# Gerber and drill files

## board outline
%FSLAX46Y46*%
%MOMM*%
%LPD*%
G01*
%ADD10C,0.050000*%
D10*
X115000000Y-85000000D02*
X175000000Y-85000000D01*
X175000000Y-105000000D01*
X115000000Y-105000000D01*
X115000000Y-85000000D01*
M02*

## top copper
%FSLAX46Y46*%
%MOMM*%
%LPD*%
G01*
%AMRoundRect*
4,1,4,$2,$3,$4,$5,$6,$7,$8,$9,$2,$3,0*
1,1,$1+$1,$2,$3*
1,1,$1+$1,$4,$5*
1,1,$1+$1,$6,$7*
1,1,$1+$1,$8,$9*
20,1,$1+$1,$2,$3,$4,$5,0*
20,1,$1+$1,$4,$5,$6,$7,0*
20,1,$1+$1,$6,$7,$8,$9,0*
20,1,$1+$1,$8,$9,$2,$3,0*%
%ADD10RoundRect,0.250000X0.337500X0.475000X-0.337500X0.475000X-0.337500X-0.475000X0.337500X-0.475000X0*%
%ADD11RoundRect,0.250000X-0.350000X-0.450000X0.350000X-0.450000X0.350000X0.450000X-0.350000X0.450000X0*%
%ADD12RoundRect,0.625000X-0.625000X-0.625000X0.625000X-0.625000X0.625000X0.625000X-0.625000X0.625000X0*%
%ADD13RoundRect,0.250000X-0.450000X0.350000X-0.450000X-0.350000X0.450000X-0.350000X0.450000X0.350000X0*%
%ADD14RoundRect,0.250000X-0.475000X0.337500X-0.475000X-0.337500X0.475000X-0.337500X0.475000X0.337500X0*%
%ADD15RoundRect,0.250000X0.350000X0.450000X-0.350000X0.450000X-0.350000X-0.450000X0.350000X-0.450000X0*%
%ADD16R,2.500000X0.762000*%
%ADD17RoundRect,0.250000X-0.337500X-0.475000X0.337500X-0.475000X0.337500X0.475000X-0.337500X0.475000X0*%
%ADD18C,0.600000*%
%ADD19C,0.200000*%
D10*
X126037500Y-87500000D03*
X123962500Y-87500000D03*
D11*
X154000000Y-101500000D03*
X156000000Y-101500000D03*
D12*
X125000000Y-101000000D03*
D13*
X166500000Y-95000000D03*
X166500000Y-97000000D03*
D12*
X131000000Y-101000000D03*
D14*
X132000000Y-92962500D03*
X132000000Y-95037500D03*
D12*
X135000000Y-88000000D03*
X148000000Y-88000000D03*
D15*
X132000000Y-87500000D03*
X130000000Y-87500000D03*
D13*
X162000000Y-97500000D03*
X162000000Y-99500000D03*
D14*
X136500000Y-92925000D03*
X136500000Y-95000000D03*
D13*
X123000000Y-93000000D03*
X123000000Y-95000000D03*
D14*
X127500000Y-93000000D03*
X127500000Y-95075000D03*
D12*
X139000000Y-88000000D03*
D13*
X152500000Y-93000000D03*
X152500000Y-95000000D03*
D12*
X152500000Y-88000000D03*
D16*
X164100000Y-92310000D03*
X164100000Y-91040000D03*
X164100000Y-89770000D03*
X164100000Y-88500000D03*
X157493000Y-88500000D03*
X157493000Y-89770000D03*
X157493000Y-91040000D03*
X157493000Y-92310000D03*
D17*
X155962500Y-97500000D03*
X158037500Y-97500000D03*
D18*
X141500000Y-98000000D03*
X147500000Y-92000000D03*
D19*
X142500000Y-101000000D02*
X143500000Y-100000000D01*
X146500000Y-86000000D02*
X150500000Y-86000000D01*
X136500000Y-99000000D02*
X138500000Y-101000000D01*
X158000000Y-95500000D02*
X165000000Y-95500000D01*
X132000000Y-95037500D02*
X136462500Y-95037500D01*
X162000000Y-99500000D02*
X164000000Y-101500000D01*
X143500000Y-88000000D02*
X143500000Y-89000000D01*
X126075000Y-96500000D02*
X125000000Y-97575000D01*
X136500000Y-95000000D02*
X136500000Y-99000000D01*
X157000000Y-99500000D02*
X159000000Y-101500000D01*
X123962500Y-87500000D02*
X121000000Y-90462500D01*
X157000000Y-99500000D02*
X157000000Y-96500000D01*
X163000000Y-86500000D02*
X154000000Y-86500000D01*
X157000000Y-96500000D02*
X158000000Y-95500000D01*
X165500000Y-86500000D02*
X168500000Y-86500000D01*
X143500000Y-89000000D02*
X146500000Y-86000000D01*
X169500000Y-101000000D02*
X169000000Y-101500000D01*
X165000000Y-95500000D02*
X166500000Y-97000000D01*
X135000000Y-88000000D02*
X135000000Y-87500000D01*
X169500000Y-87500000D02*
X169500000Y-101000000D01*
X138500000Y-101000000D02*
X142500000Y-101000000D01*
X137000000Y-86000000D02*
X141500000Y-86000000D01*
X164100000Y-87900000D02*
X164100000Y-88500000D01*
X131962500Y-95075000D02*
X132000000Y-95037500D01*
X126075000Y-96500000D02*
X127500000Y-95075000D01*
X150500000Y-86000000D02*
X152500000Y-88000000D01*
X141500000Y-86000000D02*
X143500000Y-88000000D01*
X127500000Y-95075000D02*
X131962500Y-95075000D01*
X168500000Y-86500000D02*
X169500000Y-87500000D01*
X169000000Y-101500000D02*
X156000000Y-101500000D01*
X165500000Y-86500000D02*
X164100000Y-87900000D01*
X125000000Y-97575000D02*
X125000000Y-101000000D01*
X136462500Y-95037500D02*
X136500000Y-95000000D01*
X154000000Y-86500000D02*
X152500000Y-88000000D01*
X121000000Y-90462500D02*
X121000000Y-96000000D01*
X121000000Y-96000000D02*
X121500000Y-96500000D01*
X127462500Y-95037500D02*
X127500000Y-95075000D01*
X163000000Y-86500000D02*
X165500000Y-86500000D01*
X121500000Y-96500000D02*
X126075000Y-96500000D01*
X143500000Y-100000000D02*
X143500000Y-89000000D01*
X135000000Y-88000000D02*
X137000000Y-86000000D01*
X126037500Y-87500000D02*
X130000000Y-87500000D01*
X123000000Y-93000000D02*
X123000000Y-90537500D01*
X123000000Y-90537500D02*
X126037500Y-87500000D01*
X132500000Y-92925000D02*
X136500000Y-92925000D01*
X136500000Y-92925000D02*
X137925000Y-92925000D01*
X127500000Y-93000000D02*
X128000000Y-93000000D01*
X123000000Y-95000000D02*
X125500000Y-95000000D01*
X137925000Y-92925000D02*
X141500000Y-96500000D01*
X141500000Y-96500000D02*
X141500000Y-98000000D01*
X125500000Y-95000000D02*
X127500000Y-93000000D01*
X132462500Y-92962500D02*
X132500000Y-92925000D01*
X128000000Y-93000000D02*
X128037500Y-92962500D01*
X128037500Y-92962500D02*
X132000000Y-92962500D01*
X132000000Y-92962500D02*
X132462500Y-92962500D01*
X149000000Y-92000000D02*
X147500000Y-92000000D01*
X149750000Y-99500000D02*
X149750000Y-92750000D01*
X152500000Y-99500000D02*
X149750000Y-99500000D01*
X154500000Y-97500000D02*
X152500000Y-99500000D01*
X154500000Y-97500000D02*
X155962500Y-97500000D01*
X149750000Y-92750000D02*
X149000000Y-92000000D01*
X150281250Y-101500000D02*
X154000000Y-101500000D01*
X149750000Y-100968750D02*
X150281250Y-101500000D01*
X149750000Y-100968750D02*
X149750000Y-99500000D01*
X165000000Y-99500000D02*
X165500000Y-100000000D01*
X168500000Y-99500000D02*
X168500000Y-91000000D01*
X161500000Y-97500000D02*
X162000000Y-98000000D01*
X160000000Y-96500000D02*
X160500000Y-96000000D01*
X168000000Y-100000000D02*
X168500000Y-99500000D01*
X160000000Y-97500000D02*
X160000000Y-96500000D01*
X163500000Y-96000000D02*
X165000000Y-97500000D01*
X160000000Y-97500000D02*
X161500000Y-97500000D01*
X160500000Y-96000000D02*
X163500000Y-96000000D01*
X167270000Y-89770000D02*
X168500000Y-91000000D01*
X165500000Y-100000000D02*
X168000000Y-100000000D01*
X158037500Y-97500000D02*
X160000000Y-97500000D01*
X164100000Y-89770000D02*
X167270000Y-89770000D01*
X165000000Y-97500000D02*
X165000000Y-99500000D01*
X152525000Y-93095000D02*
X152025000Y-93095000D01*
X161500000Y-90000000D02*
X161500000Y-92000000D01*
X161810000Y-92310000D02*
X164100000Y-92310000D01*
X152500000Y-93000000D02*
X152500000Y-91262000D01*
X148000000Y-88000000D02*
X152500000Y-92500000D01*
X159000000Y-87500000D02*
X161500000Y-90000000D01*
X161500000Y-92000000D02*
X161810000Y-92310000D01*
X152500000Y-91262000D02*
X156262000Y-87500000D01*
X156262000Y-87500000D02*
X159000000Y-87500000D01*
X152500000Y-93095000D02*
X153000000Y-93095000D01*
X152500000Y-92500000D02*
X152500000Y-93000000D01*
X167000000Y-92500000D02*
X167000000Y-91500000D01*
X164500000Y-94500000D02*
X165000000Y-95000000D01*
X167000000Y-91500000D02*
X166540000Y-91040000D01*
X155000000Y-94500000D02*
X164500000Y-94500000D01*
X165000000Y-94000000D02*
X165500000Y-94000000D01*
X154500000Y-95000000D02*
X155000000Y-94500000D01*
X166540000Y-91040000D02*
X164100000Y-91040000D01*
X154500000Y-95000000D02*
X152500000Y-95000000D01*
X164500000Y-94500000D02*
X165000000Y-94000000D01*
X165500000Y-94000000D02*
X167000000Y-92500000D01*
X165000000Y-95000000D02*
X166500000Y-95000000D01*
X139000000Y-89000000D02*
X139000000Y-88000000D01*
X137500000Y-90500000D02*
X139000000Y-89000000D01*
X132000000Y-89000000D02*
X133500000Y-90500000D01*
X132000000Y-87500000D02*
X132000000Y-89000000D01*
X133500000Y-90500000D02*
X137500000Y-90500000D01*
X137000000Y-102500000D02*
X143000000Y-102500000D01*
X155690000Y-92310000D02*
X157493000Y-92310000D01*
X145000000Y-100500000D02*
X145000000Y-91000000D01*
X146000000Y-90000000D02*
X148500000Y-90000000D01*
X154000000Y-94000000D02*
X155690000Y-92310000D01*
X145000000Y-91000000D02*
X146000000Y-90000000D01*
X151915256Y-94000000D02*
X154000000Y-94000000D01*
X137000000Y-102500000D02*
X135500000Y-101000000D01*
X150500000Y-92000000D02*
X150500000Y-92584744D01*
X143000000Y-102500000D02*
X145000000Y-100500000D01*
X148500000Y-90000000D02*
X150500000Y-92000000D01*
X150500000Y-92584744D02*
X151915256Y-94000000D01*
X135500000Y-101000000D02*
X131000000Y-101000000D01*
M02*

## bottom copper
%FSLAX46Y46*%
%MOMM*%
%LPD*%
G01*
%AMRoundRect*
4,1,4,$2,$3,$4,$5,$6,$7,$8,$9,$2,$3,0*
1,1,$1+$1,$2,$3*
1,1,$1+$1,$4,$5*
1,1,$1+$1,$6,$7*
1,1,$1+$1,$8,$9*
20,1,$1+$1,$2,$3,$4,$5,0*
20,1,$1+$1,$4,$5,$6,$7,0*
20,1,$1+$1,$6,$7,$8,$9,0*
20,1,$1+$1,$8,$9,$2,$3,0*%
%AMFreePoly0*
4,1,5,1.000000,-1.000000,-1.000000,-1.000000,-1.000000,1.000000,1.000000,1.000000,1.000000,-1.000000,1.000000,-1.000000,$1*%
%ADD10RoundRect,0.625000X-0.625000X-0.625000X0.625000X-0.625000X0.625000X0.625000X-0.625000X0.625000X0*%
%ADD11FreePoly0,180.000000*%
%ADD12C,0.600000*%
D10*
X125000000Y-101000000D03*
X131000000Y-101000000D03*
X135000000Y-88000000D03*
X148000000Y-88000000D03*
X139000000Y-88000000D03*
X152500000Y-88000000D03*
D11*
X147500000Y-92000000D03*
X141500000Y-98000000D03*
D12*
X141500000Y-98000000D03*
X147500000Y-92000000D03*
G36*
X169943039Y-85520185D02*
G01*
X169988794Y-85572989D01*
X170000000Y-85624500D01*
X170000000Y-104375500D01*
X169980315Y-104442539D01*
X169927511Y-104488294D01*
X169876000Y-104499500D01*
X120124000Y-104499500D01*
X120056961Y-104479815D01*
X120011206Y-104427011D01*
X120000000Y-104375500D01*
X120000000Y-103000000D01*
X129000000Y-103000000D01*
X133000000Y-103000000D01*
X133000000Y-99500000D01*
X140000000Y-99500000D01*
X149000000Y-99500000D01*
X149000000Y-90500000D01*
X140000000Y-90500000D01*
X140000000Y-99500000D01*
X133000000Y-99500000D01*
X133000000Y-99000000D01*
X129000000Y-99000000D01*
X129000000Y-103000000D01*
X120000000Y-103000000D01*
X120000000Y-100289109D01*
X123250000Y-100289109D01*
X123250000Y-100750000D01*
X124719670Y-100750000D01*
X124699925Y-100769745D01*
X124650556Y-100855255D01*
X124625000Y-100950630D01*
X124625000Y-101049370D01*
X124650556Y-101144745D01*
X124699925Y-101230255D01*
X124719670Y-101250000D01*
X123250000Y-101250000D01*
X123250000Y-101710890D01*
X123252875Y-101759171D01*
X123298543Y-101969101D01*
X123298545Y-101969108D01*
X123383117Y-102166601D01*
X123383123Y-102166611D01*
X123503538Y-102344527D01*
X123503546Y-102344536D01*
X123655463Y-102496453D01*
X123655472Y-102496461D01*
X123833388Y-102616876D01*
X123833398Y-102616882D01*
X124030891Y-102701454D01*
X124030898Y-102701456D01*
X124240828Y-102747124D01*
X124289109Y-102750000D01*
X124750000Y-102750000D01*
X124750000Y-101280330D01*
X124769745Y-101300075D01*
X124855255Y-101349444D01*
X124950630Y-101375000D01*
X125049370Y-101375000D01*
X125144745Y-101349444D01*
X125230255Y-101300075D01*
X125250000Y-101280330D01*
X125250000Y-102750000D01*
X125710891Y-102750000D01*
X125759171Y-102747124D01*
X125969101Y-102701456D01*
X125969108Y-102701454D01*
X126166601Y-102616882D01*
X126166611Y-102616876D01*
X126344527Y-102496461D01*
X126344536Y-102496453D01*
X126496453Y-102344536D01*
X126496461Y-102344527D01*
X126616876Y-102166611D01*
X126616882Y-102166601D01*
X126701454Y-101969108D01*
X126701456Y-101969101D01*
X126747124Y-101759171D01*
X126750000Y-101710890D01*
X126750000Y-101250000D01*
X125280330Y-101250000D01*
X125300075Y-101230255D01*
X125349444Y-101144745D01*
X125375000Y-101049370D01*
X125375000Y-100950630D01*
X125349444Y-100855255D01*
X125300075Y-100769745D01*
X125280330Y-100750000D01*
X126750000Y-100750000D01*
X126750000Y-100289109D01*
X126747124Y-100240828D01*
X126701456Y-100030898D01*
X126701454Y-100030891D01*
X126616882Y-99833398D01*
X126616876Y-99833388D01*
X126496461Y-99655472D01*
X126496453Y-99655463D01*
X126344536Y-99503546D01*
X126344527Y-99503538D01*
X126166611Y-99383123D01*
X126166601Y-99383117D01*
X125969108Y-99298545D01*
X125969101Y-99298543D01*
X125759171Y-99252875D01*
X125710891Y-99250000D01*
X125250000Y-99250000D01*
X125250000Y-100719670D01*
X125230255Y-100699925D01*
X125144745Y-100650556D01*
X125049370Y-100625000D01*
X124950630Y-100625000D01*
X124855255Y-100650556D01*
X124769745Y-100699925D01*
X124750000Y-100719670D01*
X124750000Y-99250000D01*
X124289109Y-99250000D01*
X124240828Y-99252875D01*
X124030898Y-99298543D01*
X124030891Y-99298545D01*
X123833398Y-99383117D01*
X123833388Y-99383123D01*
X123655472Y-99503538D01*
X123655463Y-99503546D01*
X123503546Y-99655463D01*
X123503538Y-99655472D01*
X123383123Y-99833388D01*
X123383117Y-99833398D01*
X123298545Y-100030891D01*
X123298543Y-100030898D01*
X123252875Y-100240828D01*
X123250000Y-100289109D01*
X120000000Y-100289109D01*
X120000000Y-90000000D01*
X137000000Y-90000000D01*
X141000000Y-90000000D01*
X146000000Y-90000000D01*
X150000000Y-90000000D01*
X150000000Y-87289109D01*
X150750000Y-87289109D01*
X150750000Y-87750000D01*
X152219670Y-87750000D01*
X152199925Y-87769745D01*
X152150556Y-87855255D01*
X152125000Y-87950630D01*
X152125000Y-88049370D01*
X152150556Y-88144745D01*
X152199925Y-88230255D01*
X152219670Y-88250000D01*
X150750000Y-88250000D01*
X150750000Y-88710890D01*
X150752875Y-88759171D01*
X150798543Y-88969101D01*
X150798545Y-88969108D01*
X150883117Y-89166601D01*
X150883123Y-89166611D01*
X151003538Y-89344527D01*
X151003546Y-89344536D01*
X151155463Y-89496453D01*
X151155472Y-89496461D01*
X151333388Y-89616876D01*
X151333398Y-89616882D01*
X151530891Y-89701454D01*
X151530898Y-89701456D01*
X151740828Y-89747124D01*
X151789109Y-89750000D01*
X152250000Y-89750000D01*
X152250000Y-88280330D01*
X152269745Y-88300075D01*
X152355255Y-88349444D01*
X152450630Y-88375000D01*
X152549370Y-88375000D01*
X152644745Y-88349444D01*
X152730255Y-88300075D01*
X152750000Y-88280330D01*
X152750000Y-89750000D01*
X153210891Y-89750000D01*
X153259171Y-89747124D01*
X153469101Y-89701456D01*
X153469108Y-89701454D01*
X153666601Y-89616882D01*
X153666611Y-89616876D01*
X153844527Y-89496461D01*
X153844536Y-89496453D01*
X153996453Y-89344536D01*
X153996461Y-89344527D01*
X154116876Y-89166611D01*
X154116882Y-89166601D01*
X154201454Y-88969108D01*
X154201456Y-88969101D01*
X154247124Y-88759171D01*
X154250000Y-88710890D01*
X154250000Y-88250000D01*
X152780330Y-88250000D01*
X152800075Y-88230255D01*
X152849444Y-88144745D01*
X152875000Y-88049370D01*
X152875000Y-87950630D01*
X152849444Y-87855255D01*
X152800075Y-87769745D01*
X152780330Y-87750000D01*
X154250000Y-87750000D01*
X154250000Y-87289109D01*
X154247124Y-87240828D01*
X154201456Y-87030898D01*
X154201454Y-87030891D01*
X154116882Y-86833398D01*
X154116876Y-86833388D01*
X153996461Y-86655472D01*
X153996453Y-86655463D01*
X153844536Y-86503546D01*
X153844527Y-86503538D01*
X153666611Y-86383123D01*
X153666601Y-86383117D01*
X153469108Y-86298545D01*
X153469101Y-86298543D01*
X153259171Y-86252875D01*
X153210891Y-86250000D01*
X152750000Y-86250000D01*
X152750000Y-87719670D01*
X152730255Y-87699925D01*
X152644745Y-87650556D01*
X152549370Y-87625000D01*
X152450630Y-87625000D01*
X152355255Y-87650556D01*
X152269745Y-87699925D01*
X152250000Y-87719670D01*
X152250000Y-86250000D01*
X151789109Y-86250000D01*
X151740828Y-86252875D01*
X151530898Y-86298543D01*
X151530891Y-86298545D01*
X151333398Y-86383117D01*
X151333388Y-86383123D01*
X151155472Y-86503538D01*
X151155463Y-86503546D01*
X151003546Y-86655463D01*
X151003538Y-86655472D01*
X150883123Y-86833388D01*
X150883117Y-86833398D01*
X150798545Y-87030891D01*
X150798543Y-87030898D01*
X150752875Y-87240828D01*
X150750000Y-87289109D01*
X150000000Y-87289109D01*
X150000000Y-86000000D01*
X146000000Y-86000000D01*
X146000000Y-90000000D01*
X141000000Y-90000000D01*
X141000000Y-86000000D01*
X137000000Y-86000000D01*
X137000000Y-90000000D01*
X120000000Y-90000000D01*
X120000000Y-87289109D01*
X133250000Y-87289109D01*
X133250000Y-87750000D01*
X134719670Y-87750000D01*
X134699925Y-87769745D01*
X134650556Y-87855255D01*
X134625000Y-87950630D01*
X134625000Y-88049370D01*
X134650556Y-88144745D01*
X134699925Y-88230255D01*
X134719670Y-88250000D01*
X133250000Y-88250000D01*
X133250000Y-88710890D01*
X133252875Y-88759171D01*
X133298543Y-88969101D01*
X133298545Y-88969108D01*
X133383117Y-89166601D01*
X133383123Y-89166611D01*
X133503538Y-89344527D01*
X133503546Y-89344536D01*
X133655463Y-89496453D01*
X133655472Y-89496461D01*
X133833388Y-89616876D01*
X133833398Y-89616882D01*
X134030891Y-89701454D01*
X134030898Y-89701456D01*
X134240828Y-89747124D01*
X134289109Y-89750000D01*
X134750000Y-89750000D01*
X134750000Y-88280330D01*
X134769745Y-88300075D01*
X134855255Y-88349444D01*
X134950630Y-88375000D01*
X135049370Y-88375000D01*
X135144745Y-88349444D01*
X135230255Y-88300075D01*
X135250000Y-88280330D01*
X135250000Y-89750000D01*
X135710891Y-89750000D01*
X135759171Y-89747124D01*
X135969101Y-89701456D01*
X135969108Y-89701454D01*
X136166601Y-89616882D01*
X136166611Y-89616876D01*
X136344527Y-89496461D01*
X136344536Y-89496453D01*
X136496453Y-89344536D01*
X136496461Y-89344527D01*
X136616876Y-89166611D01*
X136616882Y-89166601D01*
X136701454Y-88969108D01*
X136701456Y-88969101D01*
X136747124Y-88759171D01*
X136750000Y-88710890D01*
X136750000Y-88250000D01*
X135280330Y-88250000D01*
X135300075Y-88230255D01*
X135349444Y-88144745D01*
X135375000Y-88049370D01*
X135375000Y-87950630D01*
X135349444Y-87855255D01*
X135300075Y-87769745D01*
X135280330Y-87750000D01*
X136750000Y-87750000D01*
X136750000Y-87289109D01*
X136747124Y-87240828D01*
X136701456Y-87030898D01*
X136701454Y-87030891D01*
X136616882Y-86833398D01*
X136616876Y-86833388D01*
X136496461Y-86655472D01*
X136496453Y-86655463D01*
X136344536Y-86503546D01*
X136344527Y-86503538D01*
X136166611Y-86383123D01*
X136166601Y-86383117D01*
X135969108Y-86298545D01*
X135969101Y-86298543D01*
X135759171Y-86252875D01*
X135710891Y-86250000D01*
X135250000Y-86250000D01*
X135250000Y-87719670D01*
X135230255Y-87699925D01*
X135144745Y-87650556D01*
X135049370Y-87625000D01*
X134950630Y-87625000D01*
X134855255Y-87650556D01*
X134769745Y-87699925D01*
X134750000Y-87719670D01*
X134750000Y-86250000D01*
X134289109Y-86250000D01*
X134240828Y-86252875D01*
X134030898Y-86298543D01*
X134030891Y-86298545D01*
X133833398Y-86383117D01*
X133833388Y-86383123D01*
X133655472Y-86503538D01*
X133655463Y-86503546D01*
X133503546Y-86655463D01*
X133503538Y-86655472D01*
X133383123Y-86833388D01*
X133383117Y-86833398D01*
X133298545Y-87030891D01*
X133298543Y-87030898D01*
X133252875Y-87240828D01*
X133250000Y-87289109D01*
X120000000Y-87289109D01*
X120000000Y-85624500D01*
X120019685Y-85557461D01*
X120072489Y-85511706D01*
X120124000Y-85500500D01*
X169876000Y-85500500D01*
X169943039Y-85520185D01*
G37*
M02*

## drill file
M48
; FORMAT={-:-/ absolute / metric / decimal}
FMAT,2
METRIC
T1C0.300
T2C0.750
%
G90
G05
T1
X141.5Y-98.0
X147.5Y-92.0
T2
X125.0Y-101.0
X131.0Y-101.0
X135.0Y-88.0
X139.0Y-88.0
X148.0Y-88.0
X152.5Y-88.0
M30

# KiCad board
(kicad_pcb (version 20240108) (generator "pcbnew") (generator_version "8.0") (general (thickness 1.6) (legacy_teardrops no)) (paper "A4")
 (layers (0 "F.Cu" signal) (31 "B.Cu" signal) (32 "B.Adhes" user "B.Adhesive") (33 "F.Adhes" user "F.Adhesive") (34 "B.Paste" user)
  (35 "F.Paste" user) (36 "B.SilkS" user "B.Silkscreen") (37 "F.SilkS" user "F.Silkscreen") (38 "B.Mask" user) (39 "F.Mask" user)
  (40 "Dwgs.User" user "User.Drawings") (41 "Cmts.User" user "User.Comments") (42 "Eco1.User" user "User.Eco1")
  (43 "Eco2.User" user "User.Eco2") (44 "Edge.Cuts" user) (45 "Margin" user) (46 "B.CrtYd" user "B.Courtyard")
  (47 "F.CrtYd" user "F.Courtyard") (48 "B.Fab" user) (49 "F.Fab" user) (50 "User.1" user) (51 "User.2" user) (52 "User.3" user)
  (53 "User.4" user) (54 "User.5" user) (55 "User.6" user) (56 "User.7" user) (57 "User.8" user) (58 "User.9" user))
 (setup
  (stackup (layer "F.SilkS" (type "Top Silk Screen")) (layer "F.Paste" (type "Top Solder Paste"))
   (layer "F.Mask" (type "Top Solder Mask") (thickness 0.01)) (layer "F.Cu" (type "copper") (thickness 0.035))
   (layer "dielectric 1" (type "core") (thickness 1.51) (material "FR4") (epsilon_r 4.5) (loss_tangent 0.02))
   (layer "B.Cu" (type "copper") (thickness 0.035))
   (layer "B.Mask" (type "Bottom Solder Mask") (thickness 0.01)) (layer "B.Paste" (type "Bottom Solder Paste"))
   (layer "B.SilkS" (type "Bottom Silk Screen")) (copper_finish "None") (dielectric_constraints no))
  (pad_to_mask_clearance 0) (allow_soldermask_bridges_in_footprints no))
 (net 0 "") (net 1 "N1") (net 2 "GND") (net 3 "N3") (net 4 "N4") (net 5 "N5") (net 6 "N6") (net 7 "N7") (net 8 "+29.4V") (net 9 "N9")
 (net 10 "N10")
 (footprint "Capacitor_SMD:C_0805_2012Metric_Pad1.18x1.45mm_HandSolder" (layer "F.Cu") (at 125 87.5 180)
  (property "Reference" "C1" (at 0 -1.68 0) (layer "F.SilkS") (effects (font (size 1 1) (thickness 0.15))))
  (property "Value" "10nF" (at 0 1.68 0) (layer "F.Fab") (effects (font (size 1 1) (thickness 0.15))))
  (pad "1" smd roundrect (at -1.0375 0 180) (size 1.175 1.45) (layers "F.Cu" "F.Paste" "F.Mask") (roundrect_rratio 0.212766) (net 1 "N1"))
  (pad "2" smd roundrect (at 1.0375 0 180) (size 1.175 1.45) (layers "F.Cu" "F.Paste" "F.Mask") (roundrect_rratio 0.212766) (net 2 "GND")))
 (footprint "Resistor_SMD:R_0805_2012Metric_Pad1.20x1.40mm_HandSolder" (layer "F.Cu") (at 155 101.5)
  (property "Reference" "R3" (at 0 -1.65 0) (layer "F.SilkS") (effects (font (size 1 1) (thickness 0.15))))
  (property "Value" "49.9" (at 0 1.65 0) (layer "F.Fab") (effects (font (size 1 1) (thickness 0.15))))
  (pad "1" smd roundrect (at -1 0) (size 1.2 1.4) (layers "F.Cu" "F.Paste" "F.Mask") (roundrect_rratio 0.208333) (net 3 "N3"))
  (pad "2" smd roundrect (at 1 0) (size 1.2 1.4) (layers "F.Cu" "F.Paste" "F.Mask") (roundrect_rratio 0.208333) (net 2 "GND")))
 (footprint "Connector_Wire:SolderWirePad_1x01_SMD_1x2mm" (layer "F.Cu") (at 125 101)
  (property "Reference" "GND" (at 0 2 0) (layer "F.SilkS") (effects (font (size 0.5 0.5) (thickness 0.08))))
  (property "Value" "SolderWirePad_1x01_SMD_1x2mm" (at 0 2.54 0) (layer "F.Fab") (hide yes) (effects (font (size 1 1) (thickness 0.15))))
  (pad "1" thru_hole roundrect (at 0 0) (size 2.5 2.5) (drill 0.75) (layers "*.Cu" "*.Mask") (remove_unused_layers no)
   (roundrect_rratio 0.25) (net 2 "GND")))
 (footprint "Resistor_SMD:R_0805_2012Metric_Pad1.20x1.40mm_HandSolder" (layer "F.Cu") (at 166.5 96 -90)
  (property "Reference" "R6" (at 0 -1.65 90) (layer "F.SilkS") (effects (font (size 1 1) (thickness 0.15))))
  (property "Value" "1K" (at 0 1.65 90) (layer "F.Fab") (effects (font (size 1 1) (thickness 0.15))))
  (pad "1" smd roundrect (at -1 0 270) (size 1.2 1.4) (layers "F.Cu" "F.Paste" "F.Mask") (roundrect_rratio 0.208333) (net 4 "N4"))
  (pad "2" smd roundrect (at 1 0 270) (size 1.2 1.4) (layers "F.Cu" "F.Paste" "F.Mask") (roundrect_rratio 0.208333) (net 2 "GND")))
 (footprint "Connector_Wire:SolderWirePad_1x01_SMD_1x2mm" (layer "F.Cu") (at 131 101)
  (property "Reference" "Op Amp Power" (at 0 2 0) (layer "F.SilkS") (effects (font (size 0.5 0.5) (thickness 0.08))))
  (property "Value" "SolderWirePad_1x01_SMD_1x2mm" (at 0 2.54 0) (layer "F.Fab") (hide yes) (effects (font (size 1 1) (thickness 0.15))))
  (pad "1" thru_hole roundrect (at 0 0) (size 2.5 2.5) (drill 0.75) (layers "*.Cu" "*.Mask") (remove_unused_layers no)
   (roundrect_rratio 0.25) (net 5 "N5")))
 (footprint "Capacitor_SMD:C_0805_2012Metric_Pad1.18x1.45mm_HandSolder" (layer "F.Cu") (at 132 94 -90)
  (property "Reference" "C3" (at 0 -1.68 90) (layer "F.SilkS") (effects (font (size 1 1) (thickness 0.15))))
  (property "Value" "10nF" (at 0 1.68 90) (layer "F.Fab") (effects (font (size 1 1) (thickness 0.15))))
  (pad "1" smd roundrect (at -1.0375 0 270) (size 1.175 1.45) (layers "F.Cu" "F.Paste" "F.Mask") (roundrect_rratio 0.212766) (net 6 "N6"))
  (pad "2" smd roundrect (at 1.0375 0 270) (size 1.175 1.45) (layers "F.Cu" "F.Paste" "F.Mask") (roundrect_rratio 0.212766) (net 2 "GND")))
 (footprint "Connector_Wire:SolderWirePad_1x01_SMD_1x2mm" (layer "F.Cu") (at 135 88)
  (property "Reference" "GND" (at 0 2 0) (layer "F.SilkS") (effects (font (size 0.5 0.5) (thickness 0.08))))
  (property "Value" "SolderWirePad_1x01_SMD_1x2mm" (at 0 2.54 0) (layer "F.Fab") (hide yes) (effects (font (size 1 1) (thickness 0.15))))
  (pad "1" thru_hole roundrect (at 0 0) (size 2.5 2.5) (drill 0.75) (layers "*.Cu" "*.Mask") (remove_unused_layers no)
   (roundrect_rratio 0.25) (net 2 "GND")))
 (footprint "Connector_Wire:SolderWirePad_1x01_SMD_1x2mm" (layer "F.Cu") (at 148 88)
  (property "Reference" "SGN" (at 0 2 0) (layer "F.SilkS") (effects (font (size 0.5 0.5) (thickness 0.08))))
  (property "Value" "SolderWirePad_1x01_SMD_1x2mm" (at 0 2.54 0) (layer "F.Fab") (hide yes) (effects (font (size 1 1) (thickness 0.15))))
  (pad "1" thru_hole roundrect (at 0 0) (size 2.5 2.5) (drill 0.75) (layers "*.Cu" "*.Mask") (remove_unused_layers no)
   (roundrect_rratio 0.25) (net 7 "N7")))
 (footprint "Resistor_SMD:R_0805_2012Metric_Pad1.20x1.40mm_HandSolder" (layer "F.Cu") (at 131 87.5 180)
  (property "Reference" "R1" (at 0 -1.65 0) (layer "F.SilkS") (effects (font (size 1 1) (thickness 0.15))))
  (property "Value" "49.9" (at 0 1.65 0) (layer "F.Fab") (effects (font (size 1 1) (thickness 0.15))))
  (pad "1" smd roundrect (at -1 0 180) (size 1.2 1.4) (layers "F.Cu" "F.Paste" "F.Mask") (roundrect_rratio 0.208333) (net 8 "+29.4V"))
  (pad "2" smd roundrect (at 1 0 180) (size 1.2 1.4) (layers "F.Cu" "F.Paste" "F.Mask") (roundrect_rratio 0.208333) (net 1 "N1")))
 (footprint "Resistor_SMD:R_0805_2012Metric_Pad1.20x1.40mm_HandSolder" (layer "F.Cu") (at 162 98.5 -90)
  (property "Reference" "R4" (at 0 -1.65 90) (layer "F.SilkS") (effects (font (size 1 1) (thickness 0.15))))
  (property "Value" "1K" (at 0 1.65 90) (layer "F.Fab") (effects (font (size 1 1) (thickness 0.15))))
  (pad "1" smd roundrect (at -1 0 270) (size 1.2 1.4) (layers "F.Cu" "F.Paste" "F.Mask") (roundrect_rratio 0.208333) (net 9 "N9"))
  (pad "2" smd roundrect (at 1 0 270) (size 1.2 1.4) (layers "F.Cu" "F.Paste" "F.Mask") (roundrect_rratio 0.208333) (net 2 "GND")))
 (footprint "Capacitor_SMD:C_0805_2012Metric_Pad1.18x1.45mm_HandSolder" (layer "F.Cu") (at 136.5 93.9625 -90)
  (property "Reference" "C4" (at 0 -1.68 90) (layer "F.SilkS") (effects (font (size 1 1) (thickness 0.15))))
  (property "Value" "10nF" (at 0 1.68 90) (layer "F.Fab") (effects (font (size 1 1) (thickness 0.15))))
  (pad "1" smd roundrect (at -1.0375 0 270) (size 1.175 1.45) (layers "F.Cu" "F.Paste" "F.Mask") (roundrect_rratio 0.212766) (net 6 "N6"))
  (pad "2" smd roundrect (at 1.0375 0 270) (size 1.175 1.45) (layers "F.Cu" "F.Paste" "F.Mask") (roundrect_rratio 0.212766) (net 2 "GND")))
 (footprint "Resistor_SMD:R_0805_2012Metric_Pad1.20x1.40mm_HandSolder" (layer "F.Cu") (at 123 94 -90)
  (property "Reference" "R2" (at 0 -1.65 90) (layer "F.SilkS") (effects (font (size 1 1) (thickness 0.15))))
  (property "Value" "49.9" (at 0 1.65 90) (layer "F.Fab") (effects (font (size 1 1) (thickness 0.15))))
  (pad "1" smd roundrect (at -1 0 270) (size 1.2 1.4) (layers "F.Cu" "F.Paste" "F.Mask") (roundrect_rratio 0.208333) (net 1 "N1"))
  (pad "2" smd roundrect (at 1 0 270) (size 1.2 1.4) (layers "F.Cu" "F.Paste" "F.Mask") (roundrect_rratio 0.208333) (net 6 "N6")))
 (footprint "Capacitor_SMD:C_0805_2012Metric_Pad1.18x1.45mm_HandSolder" (layer "F.Cu") (at 127.5 94.0375 -90)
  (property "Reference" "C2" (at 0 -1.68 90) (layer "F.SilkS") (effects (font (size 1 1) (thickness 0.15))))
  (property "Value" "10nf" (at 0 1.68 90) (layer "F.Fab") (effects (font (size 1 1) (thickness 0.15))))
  (pad "1" smd roundrect (at -1.0375 0 270) (size 1.175 1.45) (layers "F.Cu" "F.Paste" "F.Mask") (roundrect_rratio 0.212766) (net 6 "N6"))
  (pad "2" smd roundrect (at 1.0375 0 270) (size 1.175 1.45) (layers "F.Cu" "F.Paste" "F.Mask") (roundrect_rratio 0.212766) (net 2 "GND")))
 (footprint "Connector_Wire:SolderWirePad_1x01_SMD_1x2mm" (layer "F.Cu") (at 139 88)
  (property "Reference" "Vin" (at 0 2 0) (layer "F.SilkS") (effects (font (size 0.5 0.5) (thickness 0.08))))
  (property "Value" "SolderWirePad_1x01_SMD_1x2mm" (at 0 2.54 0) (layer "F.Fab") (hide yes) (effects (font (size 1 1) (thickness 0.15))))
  (pad "1" thru_hole roundrect (at 0 0) (size 2.5 2.5) (drill 0.75) (layers "*.Cu" "*.Mask") (remove_unused_layers no)
   (roundrect_rratio 0.25) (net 8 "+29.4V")))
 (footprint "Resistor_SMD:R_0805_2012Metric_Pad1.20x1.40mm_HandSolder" (layer "F.Cu") (at 152.5 94 -90)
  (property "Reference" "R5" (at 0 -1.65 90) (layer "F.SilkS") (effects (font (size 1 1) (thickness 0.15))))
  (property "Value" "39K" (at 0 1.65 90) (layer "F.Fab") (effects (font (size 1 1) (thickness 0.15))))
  (pad "1" smd roundrect (at -1 0 270) (size 1.2 1.4) (layers "F.Cu" "F.Paste" "F.Mask") (roundrect_rratio 0.208333) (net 7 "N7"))
  (pad "2" smd roundrect (at 1 0 270) (size 1.2 1.4) (layers "F.Cu" "F.Paste" "F.Mask") (roundrect_rratio 0.208333) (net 4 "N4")))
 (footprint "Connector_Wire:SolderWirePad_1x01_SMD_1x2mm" (layer "F.Cu") (at 152.5 88)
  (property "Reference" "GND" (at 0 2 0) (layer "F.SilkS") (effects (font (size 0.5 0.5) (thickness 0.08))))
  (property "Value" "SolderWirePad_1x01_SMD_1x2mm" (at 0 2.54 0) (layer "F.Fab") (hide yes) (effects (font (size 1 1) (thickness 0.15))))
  (pad "1" thru_hole roundrect (at 0 0) (size 2.5 2.5) (drill 0.75) (layers "*.Cu" "*.Mask") (remove_unused_layers no)
   (roundrect_rratio 0.25) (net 2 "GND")))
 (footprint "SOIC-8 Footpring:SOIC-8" (layer "F.Cu") (at 161.5 90.405)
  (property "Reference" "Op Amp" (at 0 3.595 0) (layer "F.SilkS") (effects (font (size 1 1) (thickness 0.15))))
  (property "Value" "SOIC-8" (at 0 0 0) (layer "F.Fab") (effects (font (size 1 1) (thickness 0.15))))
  (pad "1" smd rect (at 2.6 1.905 90) (size 0.762 2.5) (layers "F.Cu" "F.Paste" "F.Mask") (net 7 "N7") (thermal_bridge_angle 45))
  (pad "2" smd rect (at 2.6 0.635 90) (size 0.762 2.5) (layers "F.Cu" "F.Paste" "F.Mask") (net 4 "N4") (thermal_bridge_angle 45))
  (pad "3" smd rect (at 2.6 -0.635 90) (size 0.762 2.5) (layers "F.Cu" "F.Paste" "F.Mask") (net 9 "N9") (thermal_bridge_angle 45))
  (pad "4" smd rect (at 2.6 -1.905 90) (size 0.762 2.5) (layers "F.Cu" "F.Paste" "F.Mask") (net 2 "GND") (thermal_bridge_angle 45))
  (pad "5" smd rect (at -4.007 -1.905 90) (size 0.762 2.5) (layers "F.Cu" "F.Paste" "F.Mask") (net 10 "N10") (thermal_bridge_angle 45))
  (pad "6" smd rect (at -4.007 -0.635 90) (size 0.762 2.5) (layers "F.Cu" "F.Paste" "F.Mask") (thermal_bridge_angle 45))
  (pad "7" smd rect (at -4.007 0.635 90) (size 0.762 2.5) (layers "F.Cu" "F.Paste" "F.Mask") (thermal_bridge_angle 45))
  (pad "8" smd rect (at -4.007 1.905 90) (size 0.762 2.5) (layers "F.Cu" "F.Paste" "F.Mask") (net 5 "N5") (thermal_bridge_angle 45)))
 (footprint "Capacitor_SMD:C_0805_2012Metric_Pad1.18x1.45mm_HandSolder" (layer "F.Cu") (at 157 97.5)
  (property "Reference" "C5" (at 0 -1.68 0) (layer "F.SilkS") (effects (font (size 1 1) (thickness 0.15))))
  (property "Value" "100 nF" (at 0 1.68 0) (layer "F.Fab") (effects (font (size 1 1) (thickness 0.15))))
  (pad "1" smd roundrect (at -1.0375 0) (size 1.175 1.45) (layers "F.Cu" "F.Paste" "F.Mask") (roundrect_rratio 0.212766) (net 3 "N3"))
  (pad "2" smd roundrect (at 1.0375 0) (size 1.175 1.45) (layers "F.Cu" "F.Paste" "F.Mask") (roundrect_rratio 0.212766) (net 9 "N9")))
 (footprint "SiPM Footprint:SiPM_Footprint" (layer "B.Cu") (at 144.5 95 180)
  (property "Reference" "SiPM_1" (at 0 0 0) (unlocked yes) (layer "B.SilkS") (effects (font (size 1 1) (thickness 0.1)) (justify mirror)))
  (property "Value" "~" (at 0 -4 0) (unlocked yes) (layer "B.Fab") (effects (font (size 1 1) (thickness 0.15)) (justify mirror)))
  (pad "1" smd custom (at -3 3 180) (size 2 2) (layers "B.Cu" "B.Paste" "B.Mask") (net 3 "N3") (thermal_bridge_angle 45)
   (options (clearance outline) (anchor rect)) (primitives))
  (pad "3" smd custom (at 3 -3 180) (size 2 2) (layers "B.Cu" "B.Paste" "B.Mask") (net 6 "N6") (thermal_bridge_angle 45)
   (options (clearance outline) (anchor rect)) (primitives)))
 (gr_rect (start 115 85) (end 175 105) (stroke (width 0.05) (type default)) (fill none) (layer "Edge.Cuts"))
 (segment (start 142.5 101) (end 143.5 100) (width 0.2) (layer "F.Cu") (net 2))
 (segment (start 146.5 86) (end 150.5 86) (width 0.2) (layer "F.Cu") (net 2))
 (segment (start 136.5 99) (end 138.5 101) (width 0.2) (layer "F.Cu") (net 2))
 (segment (start 158 95.5) (end 165 95.5) (width 0.2) (layer "F.Cu") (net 2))
 (segment (start 132 95.0375) (end 136.4625 95.0375) (width 0.2) (layer "F.Cu") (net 2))
 (segment (start 162 99.5) (end 164 101.5) (width 0.2) (layer "F.Cu") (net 2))
 (segment (start 143.5 88) (end 143.5 89) (width 0.2) (layer "F.Cu") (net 2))
 (segment (start 126.075 96.5) (end 125 97.575) (width 0.2) (layer "F.Cu") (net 2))
 (segment (start 136.5 95) (end 136.5 99) (width 0.2) (layer "F.Cu") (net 2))
 (segment (start 157 99.5) (end 159 101.5) (width 0.2) (layer "F.Cu") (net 2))
 (segment (start 123.9625 87.5) (end 121 90.4625) (width 0.2) (layer "F.Cu") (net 2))
 (segment (start 157 99.5) (end 157 96.5) (width 0.2) (layer "F.Cu") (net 2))
 (segment (start 163 86.5) (end 154 86.5) (width 0.2) (layer "F.Cu") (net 2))
 (segment (start 157 96.5) (end 158 95.5) (width 0.2) (layer "F.Cu") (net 2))
 (segment (start 165.5 86.5) (end 168.5 86.5) (width 0.2) (layer "F.Cu") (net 2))
 (segment (start 143.5 89) (end 146.5 86) (width 0.2) (layer "F.Cu") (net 2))
 (segment (start 169.5 101) (end 169 101.5) (width 0.2) (layer "F.Cu") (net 2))
 (segment (start 165 95.5) (end 166.5 97) (width 0.2) (layer "F.Cu") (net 2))
 (segment (start 135 88) (end 135 87.5) (width 0.2) (layer "F.Cu") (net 2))
 (segment (start 169.5 87.5) (end 169.5 101) (width 0.2) (layer "F.Cu") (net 2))
 (segment (start 138.5 101) (end 142.5 101) (width 0.2) (layer "F.Cu") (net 2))
 (segment (start 137 86) (end 141.5 86) (width 0.2) (layer "F.Cu") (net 2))
 (segment (start 164.1 87.9) (end 164.1 88.5) (width 0.2) (layer "F.Cu") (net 2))
 (segment (start 131.9625 95.075) (end 132 95.0375) (width 0.2) (layer "F.Cu") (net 2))
 (segment (start 126.075 96.5) (end 127.5 95.075) (width 0.2) (layer "F.Cu") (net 2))
 (segment (start 150.5 86) (end 152.5 88) (width 0.2) (layer "F.Cu") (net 2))
 (segment (start 141.5 86) (end 143.5 88) (width 0.2) (layer "F.Cu") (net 2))
 (segment (start 127.5 95.075) (end 131.9625 95.075) (width 0.2) (layer "F.Cu") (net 2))
 (segment (start 168.5 86.5) (end 169.5 87.5) (width 0.2) (layer "F.Cu") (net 2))
 (segment (start 169 101.5) (end 156 101.5) (width 0.2) (layer "F.Cu") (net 2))
 (segment (start 165.5 86.5) (end 164.1 87.9) (width 0.2) (layer "F.Cu") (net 2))
 (segment (start 125 97.575) (end 125 101) (width 0.2) (layer "F.Cu") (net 2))
 (segment (start 136.4625 95.0375) (end 136.5 95) (width 0.2) (layer "F.Cu") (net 2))
 (segment (start 154 86.5) (end 152.5 88) (width 0.2) (layer "F.Cu") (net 2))
 (segment (start 121 90.4625) (end 121 96) (width 0.2) (layer "F.Cu") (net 2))
 (segment (start 121 96) (end 121.5 96.5) (width 0.2) (layer "F.Cu") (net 2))
 (segment (start 127.4625 95.0375) (end 127.5 95.075) (width 0.2) (layer "F.Cu") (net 2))
 (segment (start 163 86.5) (end 165.5 86.5) (width 0.2) (layer "F.Cu") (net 2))
 (segment (start 121.5 96.5) (end 126.075 96.5) (width 0.2) (layer "F.Cu") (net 2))
 (segment (start 143.5 100) (end 143.5 89) (width 0.2) (layer "F.Cu") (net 2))
 (segment (start 135 88) (end 137 86) (width 0.2) (layer "F.Cu") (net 2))
 (segment (start 126.0375 87.5) (end 130 87.5) (width 0.2) (layer "F.Cu") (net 1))
 (segment (start 123 93) (end 123 90.5375) (width 0.2) (layer "F.Cu") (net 1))
 (segment (start 123 90.5375) (end 126.0375 87.5) (width 0.2) (layer "F.Cu") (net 1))
 (segment (start 132.5 92.925) (end 136.5 92.925) (width 0.2) (layer "F.Cu") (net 6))
 (segment (start 136.5 92.925) (end 137.925 92.925) (width 0.2) (layer "F.Cu") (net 6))
 (segment (start 127.5 93) (end 128 93) (width 0.2) (layer "F.Cu") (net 6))
 (segment (start 123 95) (end 125.5 95) (width 0.2) (layer "F.Cu") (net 6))
 (segment (start 137.925 92.925) (end 141.5 96.5) (width 0.2) (layer "F.Cu") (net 6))
 (segment (start 141.5 96.5) (end 141.5 98) (width 0.2) (layer "F.Cu") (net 6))
 (segment (start 125.5 95) (end 127.5 93) (width 0.2) (layer "F.Cu") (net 6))
 (segment (start 132.4625 92.9625) (end 132.5 92.925) (width 0.2) (layer "F.Cu") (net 6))
 (segment (start 128 93) (end 128.0375 92.9625) (width 0.2) (layer "F.Cu") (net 6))
 (segment (start 128.0375 92.9625) (end 132 92.9625) (width 0.2) (layer "F.Cu") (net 6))
 (segment (start 132 92.9625) (end 132.4625 92.9625) (width 0.2) (layer "F.Cu") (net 6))
 (via micro (at 141.5 98) (size 0.6) (drill 0.3) (layers "F.Cu" "B.Cu") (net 6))
 (segment (start 149 92) (end 147.5 92) (width 0.2) (layer "F.Cu") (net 3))
 (segment (start 149.75 99.5) (end 149.75 92.75) (width 0.2) (layer "F.Cu") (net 3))
 (segment (start 152.5 99.5) (end 149.75 99.5) (width 0.2) (layer "F.Cu") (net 3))
 (segment (start 154.5 97.5) (end 152.5 99.5) (width 0.2) (layer "F.Cu") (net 3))
 (segment (start 154.5 97.5) (end 155.9625 97.5) (width 0.2) (layer "F.Cu") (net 3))
 (segment (start 149.75 92.75) (end 149 92) (width 0.2) (layer "F.Cu") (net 3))
 (segment (start 150.28125 101.5) (end 154 101.5) (width 0.2) (layer "F.Cu") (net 3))
 (segment (start 149.75 100.96875) (end 150.28125 101.5) (width 0.2) (layer "F.Cu") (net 3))
 (segment (start 149.75 100.96875) (end 149.75 99.5) (width 0.2) (layer "F.Cu") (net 3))
 (via micro (at 147.5 92) (size 0.6) (drill 0.3) (layers "F.Cu" "B.Cu") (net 3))
 (segment (start 165 99.5) (end 165.5 100) (width 0.2) (layer "F.Cu") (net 9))
 (segment (start 168.5 99.5) (end 168.5 91) (width 0.2) (layer "F.Cu") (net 9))
 (segment (start 161.5 97.5) (end 162 98) (width 0.2) (layer "F.Cu") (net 9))
 (segment (start 160 96.5) (end 160.5 96) (width 0.2) (layer "F.Cu") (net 9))
 (segment (start 168 100) (end 168.5 99.5) (width 0.2) (layer "F.Cu") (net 9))
 (segment (start 160 97.5) (end 160 96.5) (width 0.2) (layer "F.Cu") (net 9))
 (segment (start 163.5 96) (end 165 97.5) (width 0.2) (layer "F.Cu") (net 9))
 (segment (start 160 97.5) (end 161.5 97.5) (width 0.2) (layer "F.Cu") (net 9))
 (segment (start 160.5 96) (end 163.5 96) (width 0.2) (layer "F.Cu") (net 9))
 (segment (start 167.27 89.77) (end 168.5 91) (width 0.2) (layer "F.Cu") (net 9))
 (segment (start 165.5 100) (end 168 100) (width 0.2) (layer "F.Cu") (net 9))
 (segment (start 158.0375 97.5) (end 160 97.5) (width 0.2) (layer "F.Cu") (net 9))
 (segment (start 164.1 89.77) (end 167.27 89.77) (width 0.2) (layer "F.Cu") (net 9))
 (segment (start 165 97.5) (end 165 99.5) (width 0.2) (layer "F.Cu") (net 9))
 (segment (start 152.525 93.095) (end 152.025 93.095) (width 0.2) (layer "F.Cu") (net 7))
 (segment (start 161.5 90) (end 161.5 92) (width 0.2) (layer "F.Cu") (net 7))
 (segment (start 161.81 92.31) (end 164.1 92.31) (width 0.2) (layer "F.Cu") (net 7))
 (segment (start 152.5 93) (end 152.5 91.262) (width 0.2) (layer "F.Cu") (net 7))
 (segment (start 148 88) (end 152.5 92.5) (width 0.2) (layer "F.Cu") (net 7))
 (segment (start 159 87.5) (end 161.5 90) (width 0.2) (layer "F.Cu") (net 7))
 (segment (start 161.5 92) (end 161.81 92.31) (width 0.2) (layer "F.Cu") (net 7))
 (segment (start 152.5 91.262) (end 156.262 87.5) (width 0.2) (layer "F.Cu") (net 7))
 (segment (start 156.262 87.5) (end 159 87.5) (width 0.2) (layer "F.Cu") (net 7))
 (segment (start 152.5 93.095) (end 153 93.095) (width 0.2) (layer "F.Cu") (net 7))
 (segment (start 152.5 92.5) (end 152.5 93) (width 0.2) (layer "F.Cu") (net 7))
 (segment (start 167 92.5) (end 167 91.5) (width 0.2) (layer "F.Cu") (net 4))
 (segment (start 164.5 94.5) (end 165 95) (width 0.2) (layer "F.Cu") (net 4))
 (segment (start 167 91.5) (end 166.54 91.04) (width 0.2) (layer "F.Cu") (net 4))
 (segment (start 155 94.5) (end 164.5 94.5) (width 0.2) (layer "F.Cu") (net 4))
 (segment (start 165 94) (end 165.5 94) (width 0.2) (layer "F.Cu") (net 4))
 (segment (start 154.5 95) (end 155 94.5) (width 0.2) (layer "F.Cu") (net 4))
 (segment (start 166.54 91.04) (end 164.1 91.04) (width 0.2) (layer "F.Cu") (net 4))
 (segment (start 154.5 95) (end 152.5 95) (width 0.2) (layer "F.Cu") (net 4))
 (segment (start 164.5 94.5) (end 165 94) (width 0.2) (layer "F.Cu") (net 4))
 (segment (start 165.5 94) (end 167 92.5) (width 0.2) (layer "F.Cu") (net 4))
 (segment (start 165 95) (end 166.5 95) (width 0.2) (layer "F.Cu") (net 4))
 (segment (start 139 89) (end 139 88) (width 0.2) (layer "F.Cu") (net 8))
 (segment (start 137.5 90.5) (end 139 89) (width 0.2) (layer "F.Cu") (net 8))
 (segment (start 132 89) (end 133.5 90.5) (width 0.2) (layer "F.Cu") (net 8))
 (segment (start 132 87.5) (end 132 89) (width 0.2) (layer "F.Cu") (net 8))
 (segment (start 133.5 90.5) (end 137.5 90.5) (width 0.2) (layer "F.Cu") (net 8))
 (segment (start 137 102.5) (end 143 102.5) (width 0.2) (layer "F.Cu") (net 5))
 (segment (start 155.69 92.31) (end 157.493 92.31) (width 0.2) (layer "F.Cu") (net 5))
 (segment (start 145 100.5) (end 145 91) (width 0.2) (layer "F.Cu") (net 5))
 (segment (start 146 90) (end 148.5 90) (width 0.2) (layer "F.Cu") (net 5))
 (segment (start 154 94) (end 155.69 92.31) (width 0.2) (layer "F.Cu") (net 5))
 (segment (start 145 91) (end 146 90) (width 0.2) (layer "F.Cu") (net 5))
 (segment (start 151.915256 94) (end 154 94) (width 0.2) (layer "F.Cu") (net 5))
 (segment (start 137 102.5) (end 135.5 101) (width 0.2) (layer "F.Cu") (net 5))
 (segment (start 150.5 92) (end 150.5 92.584744) (width 0.2) (layer "F.Cu") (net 5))
 (segment (start 143 102.5) (end 145 100.5) (width 0.2) (layer "F.Cu") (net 5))
 (segment (start 148.5 90) (end 150.5 92) (width 0.2) (layer "F.Cu") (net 5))
 (segment (start 150.5 92.584744) (end 151.915256 94) (width 0.2) (layer "F.Cu") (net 5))
 (segment (start 135.5 101) (end 131 101) (width 0.2) (layer "F.Cu") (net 5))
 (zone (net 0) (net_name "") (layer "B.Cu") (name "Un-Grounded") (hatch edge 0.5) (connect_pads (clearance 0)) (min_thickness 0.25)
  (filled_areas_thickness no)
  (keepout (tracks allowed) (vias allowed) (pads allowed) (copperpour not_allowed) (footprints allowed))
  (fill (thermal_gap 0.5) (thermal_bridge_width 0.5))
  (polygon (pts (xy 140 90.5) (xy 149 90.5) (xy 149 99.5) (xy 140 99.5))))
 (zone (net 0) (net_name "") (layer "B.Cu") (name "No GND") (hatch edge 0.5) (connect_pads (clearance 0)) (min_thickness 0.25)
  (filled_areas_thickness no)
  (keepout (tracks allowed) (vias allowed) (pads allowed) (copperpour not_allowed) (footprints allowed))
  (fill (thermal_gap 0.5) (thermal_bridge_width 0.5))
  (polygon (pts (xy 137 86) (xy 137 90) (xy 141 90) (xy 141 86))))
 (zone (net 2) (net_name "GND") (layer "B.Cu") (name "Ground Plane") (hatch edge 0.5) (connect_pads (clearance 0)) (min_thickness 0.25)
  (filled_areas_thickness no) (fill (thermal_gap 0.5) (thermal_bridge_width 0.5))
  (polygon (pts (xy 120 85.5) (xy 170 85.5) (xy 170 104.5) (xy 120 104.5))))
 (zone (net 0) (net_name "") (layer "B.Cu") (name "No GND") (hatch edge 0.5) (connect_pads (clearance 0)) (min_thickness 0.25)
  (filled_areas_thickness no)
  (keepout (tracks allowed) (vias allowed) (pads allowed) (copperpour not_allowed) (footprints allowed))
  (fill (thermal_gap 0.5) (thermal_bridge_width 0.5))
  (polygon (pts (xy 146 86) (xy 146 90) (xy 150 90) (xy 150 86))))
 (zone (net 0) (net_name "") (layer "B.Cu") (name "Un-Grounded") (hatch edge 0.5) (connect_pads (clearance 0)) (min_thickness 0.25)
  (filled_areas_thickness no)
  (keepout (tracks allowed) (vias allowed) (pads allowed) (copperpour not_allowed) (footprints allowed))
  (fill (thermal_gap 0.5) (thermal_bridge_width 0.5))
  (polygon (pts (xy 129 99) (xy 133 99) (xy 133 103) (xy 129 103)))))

